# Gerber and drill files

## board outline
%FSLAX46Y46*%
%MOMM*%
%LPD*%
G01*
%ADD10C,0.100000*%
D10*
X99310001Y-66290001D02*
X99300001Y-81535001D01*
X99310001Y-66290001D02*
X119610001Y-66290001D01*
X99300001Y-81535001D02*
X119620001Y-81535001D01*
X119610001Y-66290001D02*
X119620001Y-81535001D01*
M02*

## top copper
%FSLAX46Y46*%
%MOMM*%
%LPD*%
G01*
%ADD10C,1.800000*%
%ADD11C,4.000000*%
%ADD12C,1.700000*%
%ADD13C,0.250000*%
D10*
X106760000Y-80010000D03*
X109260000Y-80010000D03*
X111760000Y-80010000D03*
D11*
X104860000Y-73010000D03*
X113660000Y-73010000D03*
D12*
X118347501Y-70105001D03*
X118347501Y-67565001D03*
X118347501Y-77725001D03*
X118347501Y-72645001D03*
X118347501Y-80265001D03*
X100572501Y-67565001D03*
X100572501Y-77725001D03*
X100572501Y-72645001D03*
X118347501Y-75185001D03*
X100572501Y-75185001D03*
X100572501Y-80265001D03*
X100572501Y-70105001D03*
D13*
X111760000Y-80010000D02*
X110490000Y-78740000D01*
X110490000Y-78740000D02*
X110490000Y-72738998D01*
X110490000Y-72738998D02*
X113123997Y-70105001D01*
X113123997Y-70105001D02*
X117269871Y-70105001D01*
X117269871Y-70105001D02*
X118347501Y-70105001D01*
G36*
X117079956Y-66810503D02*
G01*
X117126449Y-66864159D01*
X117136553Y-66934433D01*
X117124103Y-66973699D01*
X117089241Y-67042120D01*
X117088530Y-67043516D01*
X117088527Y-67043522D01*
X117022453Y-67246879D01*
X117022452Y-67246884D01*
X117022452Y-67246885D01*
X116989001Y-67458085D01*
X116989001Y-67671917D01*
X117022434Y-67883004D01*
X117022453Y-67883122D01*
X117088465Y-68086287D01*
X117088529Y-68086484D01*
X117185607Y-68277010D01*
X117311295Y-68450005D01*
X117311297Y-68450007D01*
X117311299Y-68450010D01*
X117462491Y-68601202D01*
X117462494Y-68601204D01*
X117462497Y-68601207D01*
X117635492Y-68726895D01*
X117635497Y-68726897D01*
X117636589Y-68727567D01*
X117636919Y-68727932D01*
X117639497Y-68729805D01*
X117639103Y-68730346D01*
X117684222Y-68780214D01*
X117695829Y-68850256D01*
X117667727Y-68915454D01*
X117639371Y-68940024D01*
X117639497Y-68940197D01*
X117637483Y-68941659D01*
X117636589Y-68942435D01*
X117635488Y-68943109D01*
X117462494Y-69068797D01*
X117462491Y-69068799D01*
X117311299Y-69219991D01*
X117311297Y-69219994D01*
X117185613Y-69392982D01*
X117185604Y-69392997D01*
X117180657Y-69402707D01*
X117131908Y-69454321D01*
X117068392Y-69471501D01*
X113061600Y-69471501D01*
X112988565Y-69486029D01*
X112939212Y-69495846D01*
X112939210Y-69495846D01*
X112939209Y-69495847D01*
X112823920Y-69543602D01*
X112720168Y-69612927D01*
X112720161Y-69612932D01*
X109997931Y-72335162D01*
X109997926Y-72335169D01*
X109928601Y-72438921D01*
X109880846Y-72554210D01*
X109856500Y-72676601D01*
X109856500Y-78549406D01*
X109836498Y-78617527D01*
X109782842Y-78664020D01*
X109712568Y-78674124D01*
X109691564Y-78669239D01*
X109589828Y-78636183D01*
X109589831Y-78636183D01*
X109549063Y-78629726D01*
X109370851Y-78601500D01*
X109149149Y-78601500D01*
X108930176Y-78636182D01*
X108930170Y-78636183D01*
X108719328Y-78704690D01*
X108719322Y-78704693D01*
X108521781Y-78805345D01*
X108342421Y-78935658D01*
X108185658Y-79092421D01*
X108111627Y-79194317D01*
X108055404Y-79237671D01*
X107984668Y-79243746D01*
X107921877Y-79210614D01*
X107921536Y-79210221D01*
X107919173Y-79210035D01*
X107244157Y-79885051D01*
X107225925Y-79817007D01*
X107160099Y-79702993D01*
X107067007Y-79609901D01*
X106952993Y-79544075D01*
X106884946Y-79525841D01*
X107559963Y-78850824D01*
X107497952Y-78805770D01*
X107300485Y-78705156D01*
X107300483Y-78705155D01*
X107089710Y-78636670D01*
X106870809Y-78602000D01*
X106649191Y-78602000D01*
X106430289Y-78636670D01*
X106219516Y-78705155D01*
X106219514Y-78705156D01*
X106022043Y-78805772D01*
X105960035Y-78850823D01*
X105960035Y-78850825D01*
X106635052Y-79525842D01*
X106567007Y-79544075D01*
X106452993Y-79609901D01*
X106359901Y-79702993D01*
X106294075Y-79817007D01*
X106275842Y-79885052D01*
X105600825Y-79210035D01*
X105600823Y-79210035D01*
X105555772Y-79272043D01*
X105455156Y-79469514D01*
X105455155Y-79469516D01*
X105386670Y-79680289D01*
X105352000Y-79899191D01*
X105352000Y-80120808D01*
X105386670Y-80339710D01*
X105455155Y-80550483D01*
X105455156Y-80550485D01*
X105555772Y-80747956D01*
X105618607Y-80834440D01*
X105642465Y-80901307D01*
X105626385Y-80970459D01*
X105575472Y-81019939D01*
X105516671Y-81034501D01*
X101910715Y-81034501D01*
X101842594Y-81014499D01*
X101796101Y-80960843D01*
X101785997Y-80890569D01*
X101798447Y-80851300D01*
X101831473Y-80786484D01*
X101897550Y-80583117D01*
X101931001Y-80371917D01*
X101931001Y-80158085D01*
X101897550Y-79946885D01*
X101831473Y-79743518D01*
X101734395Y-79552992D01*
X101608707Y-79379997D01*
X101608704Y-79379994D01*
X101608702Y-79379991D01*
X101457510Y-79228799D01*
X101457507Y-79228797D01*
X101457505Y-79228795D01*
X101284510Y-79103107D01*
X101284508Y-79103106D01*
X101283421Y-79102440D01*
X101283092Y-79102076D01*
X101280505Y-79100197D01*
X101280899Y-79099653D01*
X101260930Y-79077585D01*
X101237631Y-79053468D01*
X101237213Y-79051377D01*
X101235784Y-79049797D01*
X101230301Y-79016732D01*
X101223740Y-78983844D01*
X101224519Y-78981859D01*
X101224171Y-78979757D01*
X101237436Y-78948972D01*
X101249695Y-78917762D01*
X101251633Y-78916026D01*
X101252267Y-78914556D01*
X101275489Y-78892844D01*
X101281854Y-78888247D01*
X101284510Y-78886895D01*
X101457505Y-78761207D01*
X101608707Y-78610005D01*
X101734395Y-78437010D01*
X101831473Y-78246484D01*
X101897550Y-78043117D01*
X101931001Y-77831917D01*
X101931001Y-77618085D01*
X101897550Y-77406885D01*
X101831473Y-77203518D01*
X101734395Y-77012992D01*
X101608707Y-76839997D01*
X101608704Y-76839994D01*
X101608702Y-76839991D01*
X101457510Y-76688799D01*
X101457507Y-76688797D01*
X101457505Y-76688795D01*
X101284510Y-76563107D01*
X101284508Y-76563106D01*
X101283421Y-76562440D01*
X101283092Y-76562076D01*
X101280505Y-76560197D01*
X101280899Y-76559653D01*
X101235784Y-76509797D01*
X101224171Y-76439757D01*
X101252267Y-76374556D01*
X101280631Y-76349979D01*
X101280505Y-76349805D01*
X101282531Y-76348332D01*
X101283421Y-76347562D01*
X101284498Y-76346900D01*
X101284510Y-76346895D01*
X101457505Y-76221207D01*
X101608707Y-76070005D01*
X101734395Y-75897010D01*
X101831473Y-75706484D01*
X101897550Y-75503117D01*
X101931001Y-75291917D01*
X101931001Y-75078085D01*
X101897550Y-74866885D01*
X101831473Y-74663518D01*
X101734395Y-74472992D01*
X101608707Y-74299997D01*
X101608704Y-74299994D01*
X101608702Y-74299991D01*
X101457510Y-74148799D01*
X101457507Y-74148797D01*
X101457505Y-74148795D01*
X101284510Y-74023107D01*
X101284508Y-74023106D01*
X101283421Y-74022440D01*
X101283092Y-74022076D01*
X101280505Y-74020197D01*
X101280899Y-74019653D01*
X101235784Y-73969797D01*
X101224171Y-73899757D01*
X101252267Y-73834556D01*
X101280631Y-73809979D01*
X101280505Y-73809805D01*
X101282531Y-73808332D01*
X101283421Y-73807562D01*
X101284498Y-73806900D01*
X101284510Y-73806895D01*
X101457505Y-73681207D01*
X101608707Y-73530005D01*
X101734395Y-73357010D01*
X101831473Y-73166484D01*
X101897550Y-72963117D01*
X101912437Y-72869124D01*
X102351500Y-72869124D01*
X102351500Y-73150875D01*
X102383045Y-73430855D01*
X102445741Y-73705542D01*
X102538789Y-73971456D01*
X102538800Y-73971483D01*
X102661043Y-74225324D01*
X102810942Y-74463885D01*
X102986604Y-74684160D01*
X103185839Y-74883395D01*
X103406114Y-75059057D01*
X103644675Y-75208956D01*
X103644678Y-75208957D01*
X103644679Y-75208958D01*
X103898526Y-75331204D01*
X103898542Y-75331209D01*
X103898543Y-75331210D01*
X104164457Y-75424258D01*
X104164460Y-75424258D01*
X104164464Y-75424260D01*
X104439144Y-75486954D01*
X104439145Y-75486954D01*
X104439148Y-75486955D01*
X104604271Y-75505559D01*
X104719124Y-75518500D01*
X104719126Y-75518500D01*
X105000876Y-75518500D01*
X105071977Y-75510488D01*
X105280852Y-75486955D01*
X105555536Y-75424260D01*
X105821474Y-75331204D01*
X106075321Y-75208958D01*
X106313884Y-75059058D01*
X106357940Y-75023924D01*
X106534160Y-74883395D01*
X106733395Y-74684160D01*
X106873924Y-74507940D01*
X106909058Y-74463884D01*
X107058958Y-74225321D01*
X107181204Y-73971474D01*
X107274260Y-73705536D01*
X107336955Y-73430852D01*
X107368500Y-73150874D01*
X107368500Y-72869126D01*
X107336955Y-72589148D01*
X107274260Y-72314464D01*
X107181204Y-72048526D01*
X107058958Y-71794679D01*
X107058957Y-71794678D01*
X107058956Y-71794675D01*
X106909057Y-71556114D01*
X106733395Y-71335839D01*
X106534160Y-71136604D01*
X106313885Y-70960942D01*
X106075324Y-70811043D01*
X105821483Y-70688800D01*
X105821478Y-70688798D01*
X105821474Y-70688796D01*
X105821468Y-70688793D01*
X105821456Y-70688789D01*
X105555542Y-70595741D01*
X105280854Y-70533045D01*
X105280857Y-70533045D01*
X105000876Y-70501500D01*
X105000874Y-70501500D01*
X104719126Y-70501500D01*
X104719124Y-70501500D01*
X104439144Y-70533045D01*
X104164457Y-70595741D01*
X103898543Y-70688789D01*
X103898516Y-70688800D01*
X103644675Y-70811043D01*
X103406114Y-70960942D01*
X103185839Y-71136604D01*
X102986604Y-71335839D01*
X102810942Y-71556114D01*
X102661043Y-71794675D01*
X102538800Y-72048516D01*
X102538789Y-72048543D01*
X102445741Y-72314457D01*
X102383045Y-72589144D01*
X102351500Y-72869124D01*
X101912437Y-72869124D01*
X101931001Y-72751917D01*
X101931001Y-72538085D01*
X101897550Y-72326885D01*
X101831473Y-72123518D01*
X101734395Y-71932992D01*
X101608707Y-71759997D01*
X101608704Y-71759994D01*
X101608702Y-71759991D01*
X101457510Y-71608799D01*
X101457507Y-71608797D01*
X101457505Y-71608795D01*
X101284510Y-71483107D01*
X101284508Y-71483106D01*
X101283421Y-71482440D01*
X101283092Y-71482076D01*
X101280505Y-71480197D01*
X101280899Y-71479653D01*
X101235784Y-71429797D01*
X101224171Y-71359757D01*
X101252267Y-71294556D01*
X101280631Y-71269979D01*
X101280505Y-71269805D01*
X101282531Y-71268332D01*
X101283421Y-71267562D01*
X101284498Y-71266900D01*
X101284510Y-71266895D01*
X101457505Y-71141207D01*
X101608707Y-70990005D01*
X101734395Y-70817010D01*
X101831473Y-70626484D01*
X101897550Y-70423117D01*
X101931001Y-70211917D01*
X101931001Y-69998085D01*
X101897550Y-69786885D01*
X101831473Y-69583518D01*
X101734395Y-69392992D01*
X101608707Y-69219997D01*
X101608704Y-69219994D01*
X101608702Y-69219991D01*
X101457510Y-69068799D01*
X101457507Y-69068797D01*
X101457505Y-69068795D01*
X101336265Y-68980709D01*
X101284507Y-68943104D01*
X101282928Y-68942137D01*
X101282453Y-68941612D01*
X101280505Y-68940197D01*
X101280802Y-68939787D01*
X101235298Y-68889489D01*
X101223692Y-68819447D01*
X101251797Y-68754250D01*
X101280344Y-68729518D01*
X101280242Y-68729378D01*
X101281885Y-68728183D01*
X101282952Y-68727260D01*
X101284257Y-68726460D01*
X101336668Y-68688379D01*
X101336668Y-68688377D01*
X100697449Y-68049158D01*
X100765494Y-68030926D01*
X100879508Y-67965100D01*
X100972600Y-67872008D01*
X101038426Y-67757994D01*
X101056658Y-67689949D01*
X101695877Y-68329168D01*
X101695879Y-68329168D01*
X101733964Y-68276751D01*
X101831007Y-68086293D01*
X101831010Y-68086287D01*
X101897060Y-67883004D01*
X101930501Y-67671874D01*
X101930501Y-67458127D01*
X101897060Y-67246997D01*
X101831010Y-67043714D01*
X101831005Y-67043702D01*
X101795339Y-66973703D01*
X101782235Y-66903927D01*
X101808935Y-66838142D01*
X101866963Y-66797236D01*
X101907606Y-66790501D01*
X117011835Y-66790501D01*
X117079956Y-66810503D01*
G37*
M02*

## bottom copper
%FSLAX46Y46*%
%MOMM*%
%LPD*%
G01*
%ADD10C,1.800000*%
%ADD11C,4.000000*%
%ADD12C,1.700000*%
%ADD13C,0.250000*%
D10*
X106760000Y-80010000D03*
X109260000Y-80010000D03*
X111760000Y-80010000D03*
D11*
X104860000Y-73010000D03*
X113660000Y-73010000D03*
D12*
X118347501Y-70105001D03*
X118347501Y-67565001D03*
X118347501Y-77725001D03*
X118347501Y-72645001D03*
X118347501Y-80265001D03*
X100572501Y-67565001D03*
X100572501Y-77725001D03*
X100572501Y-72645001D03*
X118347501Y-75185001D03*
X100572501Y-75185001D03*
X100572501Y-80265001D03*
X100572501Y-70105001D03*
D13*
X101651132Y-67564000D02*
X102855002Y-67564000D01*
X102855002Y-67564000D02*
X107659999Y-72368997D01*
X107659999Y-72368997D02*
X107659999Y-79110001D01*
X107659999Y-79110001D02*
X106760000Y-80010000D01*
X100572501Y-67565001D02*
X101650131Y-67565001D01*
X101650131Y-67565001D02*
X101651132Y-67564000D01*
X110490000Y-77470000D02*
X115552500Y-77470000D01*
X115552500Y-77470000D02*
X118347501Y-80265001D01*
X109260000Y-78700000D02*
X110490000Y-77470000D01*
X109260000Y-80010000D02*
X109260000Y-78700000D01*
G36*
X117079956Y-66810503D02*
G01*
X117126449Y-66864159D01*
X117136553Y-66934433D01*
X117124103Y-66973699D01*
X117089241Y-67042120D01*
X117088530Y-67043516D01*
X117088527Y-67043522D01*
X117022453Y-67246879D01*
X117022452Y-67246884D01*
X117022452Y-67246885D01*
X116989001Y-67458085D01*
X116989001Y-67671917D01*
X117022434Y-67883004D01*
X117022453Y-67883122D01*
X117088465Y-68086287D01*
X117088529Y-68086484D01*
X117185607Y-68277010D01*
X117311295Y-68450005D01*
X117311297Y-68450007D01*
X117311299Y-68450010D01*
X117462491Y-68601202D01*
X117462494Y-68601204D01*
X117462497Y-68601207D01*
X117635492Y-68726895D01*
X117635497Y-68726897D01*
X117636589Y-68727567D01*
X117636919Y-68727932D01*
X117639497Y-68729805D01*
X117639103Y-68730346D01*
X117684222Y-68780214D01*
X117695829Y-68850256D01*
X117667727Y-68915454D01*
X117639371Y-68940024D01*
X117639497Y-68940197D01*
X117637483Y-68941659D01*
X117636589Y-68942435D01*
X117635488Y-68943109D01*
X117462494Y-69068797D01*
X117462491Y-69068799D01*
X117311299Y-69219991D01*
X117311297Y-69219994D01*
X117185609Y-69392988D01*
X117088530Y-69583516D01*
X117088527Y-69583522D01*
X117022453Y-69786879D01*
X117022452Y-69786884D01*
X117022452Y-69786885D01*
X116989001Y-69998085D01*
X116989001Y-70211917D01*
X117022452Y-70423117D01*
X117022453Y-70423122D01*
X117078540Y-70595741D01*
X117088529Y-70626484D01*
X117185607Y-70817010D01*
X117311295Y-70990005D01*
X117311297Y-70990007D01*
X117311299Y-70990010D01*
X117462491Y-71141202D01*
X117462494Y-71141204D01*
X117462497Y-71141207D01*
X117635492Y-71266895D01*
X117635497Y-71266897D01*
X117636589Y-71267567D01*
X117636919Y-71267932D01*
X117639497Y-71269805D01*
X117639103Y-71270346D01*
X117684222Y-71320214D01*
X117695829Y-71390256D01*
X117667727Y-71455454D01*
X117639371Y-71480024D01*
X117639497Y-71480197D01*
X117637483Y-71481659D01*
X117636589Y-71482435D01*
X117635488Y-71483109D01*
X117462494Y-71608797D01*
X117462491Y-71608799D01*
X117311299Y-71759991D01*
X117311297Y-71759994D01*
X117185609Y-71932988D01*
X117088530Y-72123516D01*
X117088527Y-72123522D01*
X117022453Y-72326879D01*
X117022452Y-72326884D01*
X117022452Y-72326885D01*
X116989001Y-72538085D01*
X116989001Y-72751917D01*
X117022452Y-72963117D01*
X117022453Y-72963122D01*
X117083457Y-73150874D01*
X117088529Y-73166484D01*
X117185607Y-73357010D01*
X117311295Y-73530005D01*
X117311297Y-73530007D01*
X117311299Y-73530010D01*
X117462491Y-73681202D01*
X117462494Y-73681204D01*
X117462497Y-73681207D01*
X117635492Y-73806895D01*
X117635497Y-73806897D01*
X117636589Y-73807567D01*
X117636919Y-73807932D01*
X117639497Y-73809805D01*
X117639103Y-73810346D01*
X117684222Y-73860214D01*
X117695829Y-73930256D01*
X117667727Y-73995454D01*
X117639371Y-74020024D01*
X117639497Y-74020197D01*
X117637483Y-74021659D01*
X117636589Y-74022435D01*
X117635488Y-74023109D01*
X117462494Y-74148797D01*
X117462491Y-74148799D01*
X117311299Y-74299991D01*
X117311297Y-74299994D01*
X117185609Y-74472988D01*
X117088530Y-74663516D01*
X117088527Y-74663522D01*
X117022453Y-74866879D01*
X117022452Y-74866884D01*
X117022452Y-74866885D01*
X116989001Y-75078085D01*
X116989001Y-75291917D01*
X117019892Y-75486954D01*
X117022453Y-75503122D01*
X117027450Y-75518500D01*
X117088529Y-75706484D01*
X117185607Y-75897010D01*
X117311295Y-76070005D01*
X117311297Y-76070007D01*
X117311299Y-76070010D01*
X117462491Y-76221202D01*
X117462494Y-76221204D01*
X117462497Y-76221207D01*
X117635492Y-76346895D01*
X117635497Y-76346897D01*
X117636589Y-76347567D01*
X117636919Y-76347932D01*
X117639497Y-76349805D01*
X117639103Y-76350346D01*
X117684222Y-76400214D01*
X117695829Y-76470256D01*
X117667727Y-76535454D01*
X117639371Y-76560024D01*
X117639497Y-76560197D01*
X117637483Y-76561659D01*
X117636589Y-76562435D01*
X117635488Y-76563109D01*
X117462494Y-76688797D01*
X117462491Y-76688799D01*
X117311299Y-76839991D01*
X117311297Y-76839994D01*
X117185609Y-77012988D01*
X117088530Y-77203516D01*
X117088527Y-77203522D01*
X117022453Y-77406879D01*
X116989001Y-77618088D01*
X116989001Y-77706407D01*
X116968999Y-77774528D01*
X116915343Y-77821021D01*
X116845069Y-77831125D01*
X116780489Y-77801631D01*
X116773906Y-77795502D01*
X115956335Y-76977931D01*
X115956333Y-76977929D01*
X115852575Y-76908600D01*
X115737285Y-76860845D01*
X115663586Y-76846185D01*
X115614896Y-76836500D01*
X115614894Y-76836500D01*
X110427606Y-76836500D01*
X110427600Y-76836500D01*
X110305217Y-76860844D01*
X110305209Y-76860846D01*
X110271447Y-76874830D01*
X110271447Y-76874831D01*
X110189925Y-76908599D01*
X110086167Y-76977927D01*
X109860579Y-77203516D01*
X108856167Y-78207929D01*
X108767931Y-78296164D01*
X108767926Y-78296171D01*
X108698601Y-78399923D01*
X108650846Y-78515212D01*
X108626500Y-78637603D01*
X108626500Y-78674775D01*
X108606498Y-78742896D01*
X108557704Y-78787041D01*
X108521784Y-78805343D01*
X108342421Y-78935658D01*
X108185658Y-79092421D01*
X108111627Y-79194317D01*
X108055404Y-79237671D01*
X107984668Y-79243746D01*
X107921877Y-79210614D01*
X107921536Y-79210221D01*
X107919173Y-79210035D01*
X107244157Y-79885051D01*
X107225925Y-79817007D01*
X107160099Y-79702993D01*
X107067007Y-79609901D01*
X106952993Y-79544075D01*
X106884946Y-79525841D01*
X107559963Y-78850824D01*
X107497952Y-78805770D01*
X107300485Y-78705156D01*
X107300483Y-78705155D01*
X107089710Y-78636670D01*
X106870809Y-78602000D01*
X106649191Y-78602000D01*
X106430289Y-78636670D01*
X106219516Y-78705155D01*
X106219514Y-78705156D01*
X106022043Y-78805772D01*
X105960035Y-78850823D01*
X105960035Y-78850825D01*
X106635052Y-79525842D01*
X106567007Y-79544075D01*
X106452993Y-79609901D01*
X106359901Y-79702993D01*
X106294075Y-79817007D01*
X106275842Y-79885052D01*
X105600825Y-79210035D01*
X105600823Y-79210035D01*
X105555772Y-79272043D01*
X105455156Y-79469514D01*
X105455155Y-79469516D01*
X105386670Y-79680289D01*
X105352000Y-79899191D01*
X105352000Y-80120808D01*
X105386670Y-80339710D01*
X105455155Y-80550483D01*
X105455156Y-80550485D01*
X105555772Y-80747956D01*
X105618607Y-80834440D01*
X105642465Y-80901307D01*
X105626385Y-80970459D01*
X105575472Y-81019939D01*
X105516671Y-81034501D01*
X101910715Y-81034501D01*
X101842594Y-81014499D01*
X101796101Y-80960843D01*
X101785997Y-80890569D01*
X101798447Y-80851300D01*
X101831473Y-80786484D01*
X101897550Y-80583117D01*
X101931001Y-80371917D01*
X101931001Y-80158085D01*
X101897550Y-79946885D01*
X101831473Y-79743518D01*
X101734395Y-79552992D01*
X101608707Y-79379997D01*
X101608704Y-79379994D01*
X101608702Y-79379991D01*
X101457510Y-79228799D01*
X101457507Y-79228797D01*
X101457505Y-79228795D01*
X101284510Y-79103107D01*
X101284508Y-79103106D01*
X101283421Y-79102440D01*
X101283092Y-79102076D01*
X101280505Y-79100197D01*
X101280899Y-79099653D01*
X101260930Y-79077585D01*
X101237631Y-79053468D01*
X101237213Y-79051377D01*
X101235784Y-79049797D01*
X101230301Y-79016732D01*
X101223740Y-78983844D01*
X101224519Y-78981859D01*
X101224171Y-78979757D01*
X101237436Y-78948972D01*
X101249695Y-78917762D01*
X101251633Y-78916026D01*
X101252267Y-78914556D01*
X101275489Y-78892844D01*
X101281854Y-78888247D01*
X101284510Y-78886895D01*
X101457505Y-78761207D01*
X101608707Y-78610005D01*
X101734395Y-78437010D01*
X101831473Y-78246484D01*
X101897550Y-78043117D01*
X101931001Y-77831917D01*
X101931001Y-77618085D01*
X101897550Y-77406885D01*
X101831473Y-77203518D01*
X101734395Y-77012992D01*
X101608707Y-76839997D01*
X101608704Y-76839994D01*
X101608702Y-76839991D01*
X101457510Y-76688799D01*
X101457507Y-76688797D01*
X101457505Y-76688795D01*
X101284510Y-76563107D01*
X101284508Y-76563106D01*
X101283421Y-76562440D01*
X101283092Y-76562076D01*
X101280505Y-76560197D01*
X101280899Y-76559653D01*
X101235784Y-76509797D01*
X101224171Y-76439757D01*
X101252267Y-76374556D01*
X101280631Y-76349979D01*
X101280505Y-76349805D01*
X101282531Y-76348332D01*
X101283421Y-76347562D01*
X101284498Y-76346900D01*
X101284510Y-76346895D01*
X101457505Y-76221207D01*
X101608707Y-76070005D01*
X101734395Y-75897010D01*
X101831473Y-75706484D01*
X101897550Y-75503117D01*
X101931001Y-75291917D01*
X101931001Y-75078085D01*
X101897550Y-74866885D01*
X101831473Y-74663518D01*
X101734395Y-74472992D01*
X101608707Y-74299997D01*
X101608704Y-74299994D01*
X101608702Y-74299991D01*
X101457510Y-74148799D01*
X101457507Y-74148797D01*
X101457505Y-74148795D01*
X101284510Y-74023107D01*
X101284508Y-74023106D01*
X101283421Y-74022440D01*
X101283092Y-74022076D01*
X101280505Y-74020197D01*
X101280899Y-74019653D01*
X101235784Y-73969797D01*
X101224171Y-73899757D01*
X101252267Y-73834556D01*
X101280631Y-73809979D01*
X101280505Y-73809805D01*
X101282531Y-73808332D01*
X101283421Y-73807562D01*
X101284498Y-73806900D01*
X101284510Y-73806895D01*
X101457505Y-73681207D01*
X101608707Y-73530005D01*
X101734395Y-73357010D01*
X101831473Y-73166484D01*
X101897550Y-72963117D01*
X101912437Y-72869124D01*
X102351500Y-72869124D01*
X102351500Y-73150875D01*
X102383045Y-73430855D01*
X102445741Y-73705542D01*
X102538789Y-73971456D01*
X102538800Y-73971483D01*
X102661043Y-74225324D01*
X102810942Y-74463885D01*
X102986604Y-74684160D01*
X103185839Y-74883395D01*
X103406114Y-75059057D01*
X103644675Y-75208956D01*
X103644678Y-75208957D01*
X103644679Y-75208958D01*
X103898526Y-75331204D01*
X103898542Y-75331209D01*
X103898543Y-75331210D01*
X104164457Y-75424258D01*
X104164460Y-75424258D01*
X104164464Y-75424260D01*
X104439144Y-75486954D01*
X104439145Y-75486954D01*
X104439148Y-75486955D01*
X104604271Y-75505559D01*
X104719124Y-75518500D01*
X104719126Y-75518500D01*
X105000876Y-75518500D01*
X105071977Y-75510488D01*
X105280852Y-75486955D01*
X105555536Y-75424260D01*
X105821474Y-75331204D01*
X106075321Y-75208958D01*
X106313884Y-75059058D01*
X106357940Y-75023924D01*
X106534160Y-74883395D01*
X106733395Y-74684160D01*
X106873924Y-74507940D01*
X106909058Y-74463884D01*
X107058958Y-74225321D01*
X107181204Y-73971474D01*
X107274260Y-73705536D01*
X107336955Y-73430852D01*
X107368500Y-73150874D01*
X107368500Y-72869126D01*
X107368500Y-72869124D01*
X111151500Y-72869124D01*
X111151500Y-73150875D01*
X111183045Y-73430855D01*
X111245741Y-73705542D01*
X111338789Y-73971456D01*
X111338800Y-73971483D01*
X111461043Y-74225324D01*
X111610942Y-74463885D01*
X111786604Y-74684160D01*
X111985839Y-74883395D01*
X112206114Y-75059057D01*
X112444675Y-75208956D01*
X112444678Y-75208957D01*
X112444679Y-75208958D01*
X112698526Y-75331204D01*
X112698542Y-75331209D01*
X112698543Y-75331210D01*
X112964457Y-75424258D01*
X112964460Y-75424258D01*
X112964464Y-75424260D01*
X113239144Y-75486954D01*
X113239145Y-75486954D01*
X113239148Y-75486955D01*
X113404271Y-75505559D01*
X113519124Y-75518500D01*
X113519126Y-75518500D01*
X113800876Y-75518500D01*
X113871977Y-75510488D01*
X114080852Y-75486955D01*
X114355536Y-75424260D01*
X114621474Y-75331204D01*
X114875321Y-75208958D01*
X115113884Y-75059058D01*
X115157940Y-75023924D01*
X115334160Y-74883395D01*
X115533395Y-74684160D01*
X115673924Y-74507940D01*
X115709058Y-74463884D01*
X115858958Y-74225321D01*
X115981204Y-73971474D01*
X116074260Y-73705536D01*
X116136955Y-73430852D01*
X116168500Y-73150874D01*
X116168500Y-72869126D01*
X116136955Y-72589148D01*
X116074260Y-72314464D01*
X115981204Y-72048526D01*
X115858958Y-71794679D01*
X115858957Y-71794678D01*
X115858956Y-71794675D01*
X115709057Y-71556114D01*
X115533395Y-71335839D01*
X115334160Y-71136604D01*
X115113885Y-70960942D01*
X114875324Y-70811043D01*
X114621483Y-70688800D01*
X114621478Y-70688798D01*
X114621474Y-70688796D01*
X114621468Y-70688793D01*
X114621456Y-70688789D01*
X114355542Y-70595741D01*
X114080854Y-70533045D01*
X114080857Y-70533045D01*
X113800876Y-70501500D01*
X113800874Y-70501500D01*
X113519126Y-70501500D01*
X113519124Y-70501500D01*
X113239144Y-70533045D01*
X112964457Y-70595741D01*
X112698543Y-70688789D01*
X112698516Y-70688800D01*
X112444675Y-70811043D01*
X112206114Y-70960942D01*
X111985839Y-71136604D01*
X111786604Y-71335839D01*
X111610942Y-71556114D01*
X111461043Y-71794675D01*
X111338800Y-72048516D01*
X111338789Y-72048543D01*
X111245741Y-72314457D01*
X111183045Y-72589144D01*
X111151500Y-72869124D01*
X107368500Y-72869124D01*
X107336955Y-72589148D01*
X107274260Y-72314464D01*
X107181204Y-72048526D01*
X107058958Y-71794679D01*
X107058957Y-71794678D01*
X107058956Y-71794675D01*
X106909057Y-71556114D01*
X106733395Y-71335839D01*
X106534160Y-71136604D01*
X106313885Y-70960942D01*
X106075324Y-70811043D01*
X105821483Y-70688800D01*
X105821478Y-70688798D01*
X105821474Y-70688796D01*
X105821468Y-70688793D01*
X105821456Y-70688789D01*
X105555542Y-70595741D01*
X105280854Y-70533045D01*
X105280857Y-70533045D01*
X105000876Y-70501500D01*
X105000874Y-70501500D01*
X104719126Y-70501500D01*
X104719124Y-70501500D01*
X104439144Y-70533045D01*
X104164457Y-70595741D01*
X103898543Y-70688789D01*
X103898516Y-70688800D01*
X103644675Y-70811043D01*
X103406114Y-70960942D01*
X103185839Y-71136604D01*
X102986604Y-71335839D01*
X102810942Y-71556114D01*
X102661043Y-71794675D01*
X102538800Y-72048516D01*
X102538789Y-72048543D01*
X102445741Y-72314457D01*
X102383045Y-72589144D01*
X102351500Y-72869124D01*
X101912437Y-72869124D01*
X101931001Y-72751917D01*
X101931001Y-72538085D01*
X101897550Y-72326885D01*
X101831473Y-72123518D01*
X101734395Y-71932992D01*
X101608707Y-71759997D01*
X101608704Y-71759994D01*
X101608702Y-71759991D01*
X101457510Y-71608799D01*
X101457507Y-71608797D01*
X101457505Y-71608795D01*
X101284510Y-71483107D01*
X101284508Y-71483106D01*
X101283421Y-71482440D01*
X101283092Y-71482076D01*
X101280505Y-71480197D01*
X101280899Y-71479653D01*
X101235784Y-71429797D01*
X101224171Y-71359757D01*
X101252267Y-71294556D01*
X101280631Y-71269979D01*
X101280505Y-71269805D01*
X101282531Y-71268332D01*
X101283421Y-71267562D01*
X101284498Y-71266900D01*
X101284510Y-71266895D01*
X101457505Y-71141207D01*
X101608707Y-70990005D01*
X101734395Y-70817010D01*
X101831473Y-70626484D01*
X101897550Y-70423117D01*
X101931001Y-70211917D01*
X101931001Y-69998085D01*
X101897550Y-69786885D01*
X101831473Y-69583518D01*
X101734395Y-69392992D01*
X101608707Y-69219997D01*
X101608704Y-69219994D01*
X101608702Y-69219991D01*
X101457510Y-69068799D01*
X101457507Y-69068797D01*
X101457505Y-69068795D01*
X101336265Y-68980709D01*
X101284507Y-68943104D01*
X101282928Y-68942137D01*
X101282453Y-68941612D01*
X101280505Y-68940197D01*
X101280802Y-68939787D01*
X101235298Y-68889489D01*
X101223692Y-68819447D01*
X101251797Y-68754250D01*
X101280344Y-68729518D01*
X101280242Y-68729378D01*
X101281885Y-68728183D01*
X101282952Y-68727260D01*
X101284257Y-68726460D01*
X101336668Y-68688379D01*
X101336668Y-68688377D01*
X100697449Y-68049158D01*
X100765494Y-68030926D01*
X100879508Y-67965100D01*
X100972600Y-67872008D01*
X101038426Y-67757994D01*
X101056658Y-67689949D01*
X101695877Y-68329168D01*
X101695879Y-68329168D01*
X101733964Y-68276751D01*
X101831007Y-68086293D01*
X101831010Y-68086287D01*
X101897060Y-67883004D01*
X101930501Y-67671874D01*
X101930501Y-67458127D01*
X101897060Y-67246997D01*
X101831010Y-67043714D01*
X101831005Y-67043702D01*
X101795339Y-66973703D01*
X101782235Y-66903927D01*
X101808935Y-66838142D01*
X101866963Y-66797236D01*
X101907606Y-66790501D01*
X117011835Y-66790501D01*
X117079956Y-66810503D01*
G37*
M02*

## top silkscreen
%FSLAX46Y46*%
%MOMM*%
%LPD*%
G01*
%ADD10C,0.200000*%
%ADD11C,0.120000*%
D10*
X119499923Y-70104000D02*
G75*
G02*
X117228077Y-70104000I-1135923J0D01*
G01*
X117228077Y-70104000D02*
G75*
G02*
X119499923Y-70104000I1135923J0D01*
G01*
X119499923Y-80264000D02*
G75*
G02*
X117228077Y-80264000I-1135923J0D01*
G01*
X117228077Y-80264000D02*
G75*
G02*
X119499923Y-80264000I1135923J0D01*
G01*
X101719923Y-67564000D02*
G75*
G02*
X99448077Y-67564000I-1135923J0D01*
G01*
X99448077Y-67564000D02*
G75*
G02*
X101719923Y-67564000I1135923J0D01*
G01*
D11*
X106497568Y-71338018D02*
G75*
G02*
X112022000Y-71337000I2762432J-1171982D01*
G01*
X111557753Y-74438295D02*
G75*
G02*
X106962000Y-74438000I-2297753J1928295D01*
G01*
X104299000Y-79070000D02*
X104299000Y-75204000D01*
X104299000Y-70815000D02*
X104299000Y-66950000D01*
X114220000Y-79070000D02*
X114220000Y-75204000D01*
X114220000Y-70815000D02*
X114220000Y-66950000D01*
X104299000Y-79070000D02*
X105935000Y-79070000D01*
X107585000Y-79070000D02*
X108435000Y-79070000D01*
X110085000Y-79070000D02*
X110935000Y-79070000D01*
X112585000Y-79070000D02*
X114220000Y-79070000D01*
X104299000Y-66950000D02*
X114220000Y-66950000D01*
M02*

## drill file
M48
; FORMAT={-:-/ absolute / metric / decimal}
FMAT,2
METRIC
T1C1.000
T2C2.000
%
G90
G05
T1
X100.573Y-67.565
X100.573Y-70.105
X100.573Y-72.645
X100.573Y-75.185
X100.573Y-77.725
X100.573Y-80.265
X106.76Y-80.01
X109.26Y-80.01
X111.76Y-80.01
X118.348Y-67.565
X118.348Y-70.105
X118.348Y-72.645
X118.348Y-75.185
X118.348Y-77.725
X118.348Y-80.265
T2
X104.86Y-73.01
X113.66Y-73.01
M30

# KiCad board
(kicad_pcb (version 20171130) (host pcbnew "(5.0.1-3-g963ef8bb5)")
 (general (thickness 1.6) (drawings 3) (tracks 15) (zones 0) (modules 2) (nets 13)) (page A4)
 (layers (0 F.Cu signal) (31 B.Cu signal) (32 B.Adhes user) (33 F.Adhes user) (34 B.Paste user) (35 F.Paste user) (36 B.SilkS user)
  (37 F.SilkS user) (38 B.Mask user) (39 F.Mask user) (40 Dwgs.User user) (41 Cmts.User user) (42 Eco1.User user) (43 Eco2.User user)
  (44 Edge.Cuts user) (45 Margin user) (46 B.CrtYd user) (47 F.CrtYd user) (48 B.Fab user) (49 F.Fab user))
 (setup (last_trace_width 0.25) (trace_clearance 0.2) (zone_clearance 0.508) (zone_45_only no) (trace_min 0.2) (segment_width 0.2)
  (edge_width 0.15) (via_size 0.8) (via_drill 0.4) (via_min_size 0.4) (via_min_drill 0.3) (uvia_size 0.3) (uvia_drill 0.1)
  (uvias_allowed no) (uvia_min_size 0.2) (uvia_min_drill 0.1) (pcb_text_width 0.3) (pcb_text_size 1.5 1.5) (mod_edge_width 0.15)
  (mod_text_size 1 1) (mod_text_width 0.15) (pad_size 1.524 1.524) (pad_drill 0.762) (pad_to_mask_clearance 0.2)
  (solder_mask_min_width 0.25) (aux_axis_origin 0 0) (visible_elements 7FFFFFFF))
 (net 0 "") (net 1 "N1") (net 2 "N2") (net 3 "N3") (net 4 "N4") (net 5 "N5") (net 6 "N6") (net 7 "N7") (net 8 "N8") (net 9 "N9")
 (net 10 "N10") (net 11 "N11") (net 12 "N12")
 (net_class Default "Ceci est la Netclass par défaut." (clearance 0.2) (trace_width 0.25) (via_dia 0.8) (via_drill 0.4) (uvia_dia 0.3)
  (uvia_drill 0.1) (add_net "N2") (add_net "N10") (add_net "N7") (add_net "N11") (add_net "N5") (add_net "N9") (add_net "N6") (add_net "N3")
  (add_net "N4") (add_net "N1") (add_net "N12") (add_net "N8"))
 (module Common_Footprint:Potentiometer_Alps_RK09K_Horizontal (layer F.Cu) (at 111.76 80.01 90)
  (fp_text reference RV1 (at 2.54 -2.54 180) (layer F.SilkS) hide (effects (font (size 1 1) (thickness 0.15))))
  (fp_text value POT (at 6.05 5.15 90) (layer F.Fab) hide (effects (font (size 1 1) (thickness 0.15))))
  (fp_arc (start 7.5 -2.5) (end 8.673 0.262) (angle -134) (layer F.SilkS) (width 0.12))
  (fp_arc (start 7.5 -2.5) (end 5.572 -4.798) (angle -100) (layer F.SilkS) (width 0.12))
  (fp_line (start 0.94 -7.461) (end 4.806 -7.461) (layer F.SilkS) (width 0.12))
  (fp_line (start 9.195 -7.461) (end 13.06 -7.461) (layer F.SilkS) (width 0.12))
  (fp_line (start 0.94 2.46) (end 4.806 2.46) (layer F.SilkS) (width 0.12))
  (fp_line (start 9.195 2.46) (end 13.06 2.46) (layer F.SilkS) (width 0.12))
  (fp_line (start 0.94 -7.461) (end 0.94 -5.825) (layer F.SilkS) (width 0.12))
  (fp_line (start 0.94 -4.175) (end 0.94 -3.325) (layer F.SilkS) (width 0.12))
  (fp_line (start 0.94 -1.675) (end 0.94 -0.825) (layer F.SilkS) (width 0.12))
  (fp_line (start 0.94 0.825) (end 0.94 2.46) (layer F.SilkS) (width 0.12))
  (fp_line (start 13.06 -7.461) (end 13.06 2.46) (layer F.SilkS) (width 0.12))
  (pad 3 thru_hole circle (at 0 -5 90) (size 1.8 1.8) (drill 1) (layers *.Cu *.Mask) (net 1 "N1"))
  (pad 2 thru_hole circle (at 0 -2.5 90) (size 1.8 1.8) (drill 1) (layers *.Cu *.Mask) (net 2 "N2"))
  (pad 1 thru_hole circle (at 0 0 90) (size 1.8 1.8) (drill 1) (layers *.Cu *.Mask) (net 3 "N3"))
  (pad 0 np_thru_hole circle (at 7 -6.9 90) (size 4 4) (drill 2) (layers *.Cu *.Mask))
  (pad 0 np_thru_hole circle (at 7 1.9 90) (size 4 4) (drill 2) (layers *.Cu *.Mask)))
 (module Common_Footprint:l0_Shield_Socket (layer F.Cu) (at 109.460001 73.915001)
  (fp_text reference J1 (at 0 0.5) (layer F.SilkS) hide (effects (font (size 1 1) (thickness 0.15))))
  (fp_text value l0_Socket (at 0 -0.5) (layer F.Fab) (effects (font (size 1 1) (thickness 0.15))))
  (fp_line (start -10.15 -7.625) (end -10.16 7.62) (layer Edge.Cuts) (width 0.1))
  (fp_line (start -10.15 -7.625) (end 10.15 -7.625) (layer Edge.Cuts) (width 0.1))
  (fp_line (start -10.16 7.62) (end 10.16 7.62) (layer Edge.Cuts) (width 0.1))
  (fp_line (start 10.15 -7.625) (end 10.16 7.62) (layer Edge.Cuts) (width 0.1))
  (pad 5 thru_hole circle (at 8.8875 -3.81 270) (size 1.7 1.7) (drill 1) (layers *.Cu *.Mask) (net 3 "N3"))
  (pad 6 thru_hole circle (at 8.8875 -6.35 270) (size 1.7 1.7) (drill 1) (layers *.Cu *.Mask) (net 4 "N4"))
  (pad 2 thru_hole circle (at 8.8875 3.81 270) (size 1.7 1.7) (drill 1) (layers *.Cu *.Mask) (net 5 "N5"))
  (pad 4 thru_hole circle (at 8.8875 -1.27 270) (size 1.7 1.7) (drill 1) (layers *.Cu *.Mask) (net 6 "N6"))
  (pad 1 thru_hole circle (at 8.8875 6.35 270) (size 1.7 1.7) (drill 1) (layers *.Cu *.Mask) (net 2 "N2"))
  (pad 7 thru_hole circle (at -8.8875 -6.35 270) (size 1.7 1.7) (drill 1) (layers *.Cu *.Mask) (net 1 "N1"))
  (pad 11 thru_hole circle (at -8.8875 3.81 270) (size 1.7 1.7) (drill 1) (layers *.Cu *.Mask) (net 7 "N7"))
  (pad 9 thru_hole circle (at -8.8875 -1.27 270) (size 1.7 1.7) (drill 1) (layers *.Cu *.Mask) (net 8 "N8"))
  (pad 3 thru_hole circle (at 8.8875 1.27 270) (size 1.7 1.7) (drill 1) (layers *.Cu *.Mask) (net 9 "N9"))
  (pad 10 thru_hole circle (at -8.8875 1.27 270) (size 1.7 1.7) (drill 1) (layers *.Cu *.Mask) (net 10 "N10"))
  (pad 12 thru_hole circle (at -8.8875 6.35 270) (size 1.7 1.7) (drill 1) (layers *.Cu *.Mask) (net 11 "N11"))
  (pad 8 thru_hole circle (at -8.8875 -3.81 270) (size 1.7 1.7) (drill 1) (layers *.Cu *.Mask) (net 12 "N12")))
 (gr_circle (center 118.364 70.104) (end 119.38 70.612) (layer F.SilkS) (width 0.2))
 (gr_circle (center 118.364 80.264) (end 119.38 80.772) (layer F.SilkS) (width 0.2))
 (gr_circle (center 100.584 67.564) (end 101.6 68.072) (layer F.SilkS) (width 0.2))
 (segment (start 101.651132 67.564) (end 102.855002 67.564) (width 0.25) (layer B.Cu) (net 1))
 (segment (start 102.855002 67.564) (end 107.659999 72.368997) (width 0.25) (layer B.Cu) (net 1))
 (segment (start 107.659999 72.368997) (end 107.659999 79.110001) (width 0.25) (layer B.Cu) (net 1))
 (segment (start 107.659999 79.110001) (end 106.76 80.01) (width 0.25) (layer B.Cu) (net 1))
 (segment (start 100.572501 67.565001) (end 101.650131 67.565001) (width 0.25) (layer B.Cu) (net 1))
 (segment (start 101.650131 67.565001) (end 101.651132 67.564) (width 0.25) (layer B.Cu) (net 1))
 (segment (start 110.49 77.47) (end 115.5525 77.47) (width 0.25) (layer B.Cu) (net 2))
 (segment (start 115.5525 77.47) (end 118.347501 80.265001) (width 0.25) (layer B.Cu) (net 2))
 (segment (start 109.26 78.7) (end 110.49 77.47) (width 0.25) (layer B.Cu) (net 2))
 (segment (start 109.26 80.01) (end 109.26 78.7) (width 0.25) (layer B.Cu) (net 2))
 (segment (start 111.76 80.01) (end 110.49 78.74) (width 0.25) (layer F.Cu) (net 3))
 (segment (start 110.49 78.74) (end 110.49 72.738998) (width 0.25) (layer F.Cu) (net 3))
 (segment (start 110.49 72.738998) (end 113.123997 70.105001) (width 0.25) (layer F.Cu) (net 3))
 (segment (start 113.123997 70.105001) (end 117.269871 70.105001) (width 0.25) (layer F.Cu) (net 3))
 (segment (start 117.269871 70.105001) (end 118.347501 70.105001) (width 0.25) (layer F.Cu) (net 3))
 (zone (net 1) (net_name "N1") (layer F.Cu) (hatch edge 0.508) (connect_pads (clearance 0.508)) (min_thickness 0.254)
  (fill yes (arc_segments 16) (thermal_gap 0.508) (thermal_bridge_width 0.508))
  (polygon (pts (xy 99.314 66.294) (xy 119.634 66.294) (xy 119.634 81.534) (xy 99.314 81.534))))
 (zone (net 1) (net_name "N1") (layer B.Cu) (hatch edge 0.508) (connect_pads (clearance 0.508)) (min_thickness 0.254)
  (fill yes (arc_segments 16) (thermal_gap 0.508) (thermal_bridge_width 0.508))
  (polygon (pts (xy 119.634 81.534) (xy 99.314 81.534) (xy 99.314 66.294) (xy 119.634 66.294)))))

